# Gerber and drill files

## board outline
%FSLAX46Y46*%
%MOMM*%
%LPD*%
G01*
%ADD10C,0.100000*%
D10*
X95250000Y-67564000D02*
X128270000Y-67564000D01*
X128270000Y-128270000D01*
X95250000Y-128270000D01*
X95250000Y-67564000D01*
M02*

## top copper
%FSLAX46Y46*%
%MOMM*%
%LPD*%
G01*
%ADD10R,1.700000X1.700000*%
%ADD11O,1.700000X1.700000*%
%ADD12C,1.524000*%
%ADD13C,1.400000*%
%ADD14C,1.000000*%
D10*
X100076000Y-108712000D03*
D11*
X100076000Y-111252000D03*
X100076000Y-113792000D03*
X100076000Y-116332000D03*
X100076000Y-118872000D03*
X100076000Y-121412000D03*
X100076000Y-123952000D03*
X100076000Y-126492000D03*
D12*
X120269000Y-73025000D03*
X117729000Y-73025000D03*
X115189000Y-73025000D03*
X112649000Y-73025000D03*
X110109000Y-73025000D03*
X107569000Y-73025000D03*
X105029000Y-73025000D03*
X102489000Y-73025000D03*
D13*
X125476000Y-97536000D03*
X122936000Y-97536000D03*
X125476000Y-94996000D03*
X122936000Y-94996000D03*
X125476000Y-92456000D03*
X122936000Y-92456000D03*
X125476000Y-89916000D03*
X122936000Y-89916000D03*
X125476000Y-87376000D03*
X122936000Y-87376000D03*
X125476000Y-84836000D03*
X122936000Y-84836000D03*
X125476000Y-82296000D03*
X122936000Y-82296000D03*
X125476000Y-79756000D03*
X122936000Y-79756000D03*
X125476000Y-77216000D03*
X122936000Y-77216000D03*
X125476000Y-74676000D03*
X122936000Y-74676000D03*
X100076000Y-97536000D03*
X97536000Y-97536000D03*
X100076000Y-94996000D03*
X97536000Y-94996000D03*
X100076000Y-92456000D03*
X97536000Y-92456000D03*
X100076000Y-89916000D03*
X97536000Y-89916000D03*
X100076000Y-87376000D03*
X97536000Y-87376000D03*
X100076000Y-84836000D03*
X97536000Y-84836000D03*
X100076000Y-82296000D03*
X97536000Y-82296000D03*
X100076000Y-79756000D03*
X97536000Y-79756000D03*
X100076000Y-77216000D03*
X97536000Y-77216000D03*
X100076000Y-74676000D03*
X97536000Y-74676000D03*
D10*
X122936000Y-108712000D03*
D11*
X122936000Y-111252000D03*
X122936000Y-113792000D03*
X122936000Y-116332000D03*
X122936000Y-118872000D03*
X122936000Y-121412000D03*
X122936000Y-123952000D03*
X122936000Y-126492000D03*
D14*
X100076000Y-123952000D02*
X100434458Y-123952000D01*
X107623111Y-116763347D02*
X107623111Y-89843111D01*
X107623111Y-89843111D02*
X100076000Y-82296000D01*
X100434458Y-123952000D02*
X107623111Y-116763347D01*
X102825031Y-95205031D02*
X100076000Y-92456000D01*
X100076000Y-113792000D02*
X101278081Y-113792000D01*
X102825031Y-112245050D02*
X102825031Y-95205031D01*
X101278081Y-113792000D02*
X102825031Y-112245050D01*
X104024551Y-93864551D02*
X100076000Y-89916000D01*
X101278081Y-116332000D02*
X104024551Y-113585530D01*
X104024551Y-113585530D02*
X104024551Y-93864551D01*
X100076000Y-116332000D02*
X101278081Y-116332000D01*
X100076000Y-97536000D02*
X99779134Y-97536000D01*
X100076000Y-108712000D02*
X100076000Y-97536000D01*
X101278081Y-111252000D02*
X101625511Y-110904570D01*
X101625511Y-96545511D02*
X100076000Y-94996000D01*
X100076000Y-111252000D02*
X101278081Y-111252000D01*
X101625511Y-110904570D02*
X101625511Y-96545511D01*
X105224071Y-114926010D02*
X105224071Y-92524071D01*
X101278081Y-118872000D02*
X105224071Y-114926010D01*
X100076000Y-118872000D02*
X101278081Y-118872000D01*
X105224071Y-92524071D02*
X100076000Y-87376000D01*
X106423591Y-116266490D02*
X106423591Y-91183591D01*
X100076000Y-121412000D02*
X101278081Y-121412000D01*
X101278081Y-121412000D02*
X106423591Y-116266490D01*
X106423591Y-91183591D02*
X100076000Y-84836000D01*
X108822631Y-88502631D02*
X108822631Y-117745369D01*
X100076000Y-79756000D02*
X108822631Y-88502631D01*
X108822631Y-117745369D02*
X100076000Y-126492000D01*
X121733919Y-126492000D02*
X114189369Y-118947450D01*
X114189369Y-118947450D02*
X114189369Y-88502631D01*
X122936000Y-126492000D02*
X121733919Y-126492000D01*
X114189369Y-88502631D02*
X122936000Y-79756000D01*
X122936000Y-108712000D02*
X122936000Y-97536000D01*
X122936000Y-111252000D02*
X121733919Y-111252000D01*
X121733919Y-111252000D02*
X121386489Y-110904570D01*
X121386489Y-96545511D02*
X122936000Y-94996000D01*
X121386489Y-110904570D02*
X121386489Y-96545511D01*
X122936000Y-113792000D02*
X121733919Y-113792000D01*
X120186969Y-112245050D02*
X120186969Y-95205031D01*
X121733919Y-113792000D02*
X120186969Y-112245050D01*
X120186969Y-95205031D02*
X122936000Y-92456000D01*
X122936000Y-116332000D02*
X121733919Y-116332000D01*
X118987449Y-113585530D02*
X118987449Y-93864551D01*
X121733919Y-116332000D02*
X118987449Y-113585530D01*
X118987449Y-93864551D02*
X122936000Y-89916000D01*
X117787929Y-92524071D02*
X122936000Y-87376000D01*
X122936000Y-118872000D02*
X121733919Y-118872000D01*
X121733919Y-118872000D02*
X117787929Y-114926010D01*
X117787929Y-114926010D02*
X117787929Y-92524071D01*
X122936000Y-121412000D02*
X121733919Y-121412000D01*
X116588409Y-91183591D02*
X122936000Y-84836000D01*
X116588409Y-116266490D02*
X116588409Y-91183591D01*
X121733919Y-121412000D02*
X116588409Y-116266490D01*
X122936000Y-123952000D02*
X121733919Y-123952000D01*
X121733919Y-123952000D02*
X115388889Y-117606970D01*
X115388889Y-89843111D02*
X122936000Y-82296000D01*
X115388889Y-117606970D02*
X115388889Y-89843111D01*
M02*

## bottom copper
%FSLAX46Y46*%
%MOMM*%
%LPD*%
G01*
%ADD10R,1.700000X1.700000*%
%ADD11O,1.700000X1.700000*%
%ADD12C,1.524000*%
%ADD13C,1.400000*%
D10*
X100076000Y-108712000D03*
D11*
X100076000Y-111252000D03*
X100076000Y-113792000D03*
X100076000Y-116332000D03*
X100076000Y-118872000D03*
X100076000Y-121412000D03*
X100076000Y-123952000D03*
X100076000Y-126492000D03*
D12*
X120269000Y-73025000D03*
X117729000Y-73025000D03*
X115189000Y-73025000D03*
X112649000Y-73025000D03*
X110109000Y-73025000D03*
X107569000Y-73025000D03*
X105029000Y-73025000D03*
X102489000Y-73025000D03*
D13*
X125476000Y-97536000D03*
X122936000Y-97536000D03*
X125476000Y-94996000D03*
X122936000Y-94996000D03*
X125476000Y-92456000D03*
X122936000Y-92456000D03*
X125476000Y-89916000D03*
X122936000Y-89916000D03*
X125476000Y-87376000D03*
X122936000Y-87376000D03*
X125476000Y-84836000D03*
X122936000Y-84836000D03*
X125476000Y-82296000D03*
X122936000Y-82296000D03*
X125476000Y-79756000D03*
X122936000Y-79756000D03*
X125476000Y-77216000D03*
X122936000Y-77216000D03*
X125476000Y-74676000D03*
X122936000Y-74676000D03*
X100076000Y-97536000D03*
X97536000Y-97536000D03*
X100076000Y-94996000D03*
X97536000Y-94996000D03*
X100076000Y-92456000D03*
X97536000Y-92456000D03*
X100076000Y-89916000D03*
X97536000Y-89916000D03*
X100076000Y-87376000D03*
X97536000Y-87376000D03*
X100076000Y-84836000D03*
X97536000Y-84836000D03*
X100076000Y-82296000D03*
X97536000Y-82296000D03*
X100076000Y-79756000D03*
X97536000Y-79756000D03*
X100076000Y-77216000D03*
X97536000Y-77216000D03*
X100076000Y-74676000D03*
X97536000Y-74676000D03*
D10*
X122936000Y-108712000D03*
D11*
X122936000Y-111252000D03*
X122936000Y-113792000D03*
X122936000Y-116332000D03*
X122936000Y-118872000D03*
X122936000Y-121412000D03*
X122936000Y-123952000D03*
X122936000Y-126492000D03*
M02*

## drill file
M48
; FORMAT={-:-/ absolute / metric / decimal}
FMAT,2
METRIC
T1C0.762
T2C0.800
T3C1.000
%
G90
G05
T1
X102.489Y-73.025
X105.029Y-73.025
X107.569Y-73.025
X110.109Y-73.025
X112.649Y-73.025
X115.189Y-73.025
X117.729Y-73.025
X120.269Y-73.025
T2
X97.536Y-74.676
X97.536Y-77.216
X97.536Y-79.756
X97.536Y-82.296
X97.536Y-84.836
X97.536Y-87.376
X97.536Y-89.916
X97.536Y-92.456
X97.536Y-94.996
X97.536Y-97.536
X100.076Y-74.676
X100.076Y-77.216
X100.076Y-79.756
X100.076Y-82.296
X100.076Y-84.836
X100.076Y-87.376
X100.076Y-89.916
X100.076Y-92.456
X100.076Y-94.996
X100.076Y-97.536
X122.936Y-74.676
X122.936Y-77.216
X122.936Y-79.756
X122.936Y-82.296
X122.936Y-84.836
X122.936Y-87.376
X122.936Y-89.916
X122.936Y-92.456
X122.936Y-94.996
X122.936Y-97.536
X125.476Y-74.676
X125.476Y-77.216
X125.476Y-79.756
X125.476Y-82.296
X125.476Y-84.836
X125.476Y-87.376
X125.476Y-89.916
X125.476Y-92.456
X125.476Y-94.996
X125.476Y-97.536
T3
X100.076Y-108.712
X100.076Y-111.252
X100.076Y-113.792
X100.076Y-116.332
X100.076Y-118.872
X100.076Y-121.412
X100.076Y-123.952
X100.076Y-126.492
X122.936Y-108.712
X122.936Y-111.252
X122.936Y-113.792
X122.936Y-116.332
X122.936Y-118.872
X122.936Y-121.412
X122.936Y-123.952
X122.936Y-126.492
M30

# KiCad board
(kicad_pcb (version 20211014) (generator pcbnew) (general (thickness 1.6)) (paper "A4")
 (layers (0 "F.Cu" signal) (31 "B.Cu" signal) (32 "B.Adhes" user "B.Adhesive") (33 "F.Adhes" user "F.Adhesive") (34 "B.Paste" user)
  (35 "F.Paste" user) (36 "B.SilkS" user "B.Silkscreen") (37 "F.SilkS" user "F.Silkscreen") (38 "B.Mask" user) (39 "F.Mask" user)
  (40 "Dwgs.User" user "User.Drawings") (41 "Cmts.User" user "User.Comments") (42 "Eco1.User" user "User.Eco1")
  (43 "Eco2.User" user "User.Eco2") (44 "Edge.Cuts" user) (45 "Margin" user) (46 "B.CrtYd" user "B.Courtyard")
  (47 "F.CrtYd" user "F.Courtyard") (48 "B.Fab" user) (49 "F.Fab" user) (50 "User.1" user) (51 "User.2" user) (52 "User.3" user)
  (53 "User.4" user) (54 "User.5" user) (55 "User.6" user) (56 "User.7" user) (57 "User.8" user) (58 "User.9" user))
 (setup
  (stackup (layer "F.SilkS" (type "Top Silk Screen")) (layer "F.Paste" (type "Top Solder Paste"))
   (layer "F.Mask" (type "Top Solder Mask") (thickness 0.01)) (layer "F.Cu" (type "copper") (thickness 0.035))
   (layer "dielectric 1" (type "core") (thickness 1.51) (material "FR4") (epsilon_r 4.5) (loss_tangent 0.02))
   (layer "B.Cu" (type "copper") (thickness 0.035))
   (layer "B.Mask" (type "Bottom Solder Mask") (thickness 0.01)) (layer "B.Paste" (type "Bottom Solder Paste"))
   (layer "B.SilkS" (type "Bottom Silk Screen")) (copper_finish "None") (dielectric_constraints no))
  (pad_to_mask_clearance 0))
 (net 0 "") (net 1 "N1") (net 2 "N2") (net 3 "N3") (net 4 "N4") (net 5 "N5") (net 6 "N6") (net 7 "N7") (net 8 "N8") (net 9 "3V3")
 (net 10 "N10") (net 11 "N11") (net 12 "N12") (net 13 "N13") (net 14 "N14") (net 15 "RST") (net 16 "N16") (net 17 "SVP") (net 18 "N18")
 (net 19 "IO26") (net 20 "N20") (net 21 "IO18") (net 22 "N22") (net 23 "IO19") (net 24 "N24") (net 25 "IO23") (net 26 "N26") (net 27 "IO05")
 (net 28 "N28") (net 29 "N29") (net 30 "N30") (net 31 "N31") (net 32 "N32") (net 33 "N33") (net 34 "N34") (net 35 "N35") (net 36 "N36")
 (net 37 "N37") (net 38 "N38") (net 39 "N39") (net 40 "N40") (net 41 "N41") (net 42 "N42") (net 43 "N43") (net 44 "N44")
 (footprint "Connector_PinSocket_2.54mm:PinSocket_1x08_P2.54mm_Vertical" (layer "F.Cu") (at 100.076 108.712)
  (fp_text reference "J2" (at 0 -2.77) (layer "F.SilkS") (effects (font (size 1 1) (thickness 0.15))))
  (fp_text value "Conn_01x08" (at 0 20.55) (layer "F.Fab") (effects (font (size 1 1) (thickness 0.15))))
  (pad "1" thru_hole rect (at 0 0) (size 1.7 1.7) (drill 1) (layers *.Cu *.Mask) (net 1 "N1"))
  (pad "2" thru_hole oval (at 0 2.54) (size 1.7 1.7) (drill 1) (layers *.Cu *.Mask) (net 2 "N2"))
  (pad "3" thru_hole oval (at 0 5.08) (size 1.7 1.7) (drill 1) (layers *.Cu *.Mask) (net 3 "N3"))
  (pad "4" thru_hole oval (at 0 7.62) (size 1.7 1.7) (drill 1) (layers *.Cu *.Mask) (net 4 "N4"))
  (pad "5" thru_hole oval (at 0 10.16) (size 1.7 1.7) (drill 1) (layers *.Cu *.Mask) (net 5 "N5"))
  (pad "6" thru_hole oval (at 0 12.7) (size 1.7 1.7) (drill 1) (layers *.Cu *.Mask) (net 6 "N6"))
  (pad "7" thru_hole oval (at 0 15.24) (size 1.7 1.7) (drill 1) (layers *.Cu *.Mask) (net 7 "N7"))
  (pad "8" thru_hole oval (at 0 17.78) (size 1.7 1.7) (drill 1) (layers *.Cu *.Mask) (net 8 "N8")))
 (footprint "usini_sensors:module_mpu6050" (layer "F.Cu") (at 102.489 73.025 -90)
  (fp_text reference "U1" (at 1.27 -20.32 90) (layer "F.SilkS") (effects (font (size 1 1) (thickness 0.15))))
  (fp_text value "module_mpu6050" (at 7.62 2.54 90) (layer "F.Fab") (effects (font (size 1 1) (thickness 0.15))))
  (pad "1" thru_hole circle locked (at 0 -17.78 270) (size 1.524 1.524) (drill 0.762) (layers *.Cu *.Mask) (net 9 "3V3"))
  (pad "2" thru_hole circle locked (at 0 -15.24 270) (size 1.524 1.524) (drill 0.762) (layers *.Cu *.Mask) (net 7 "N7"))
  (pad "3" thru_hole circle locked (at 0 -12.7 270) (size 1.524 1.524) (drill 0.762) (layers *.Cu *.Mask) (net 3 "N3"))
  (pad "4" thru_hole circle locked (at 0 -10.16 270) (size 1.524 1.524) (drill 0.762) (layers *.Cu *.Mask) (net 4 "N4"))
  (pad "5" thru_hole circle locked (at 0 -7.62 270) (size 1.524 1.524) (drill 0.762) (layers *.Cu *.Mask) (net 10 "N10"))
  (pad "6" thru_hole circle locked (at 0 -5.08 270) (size 1.524 1.524) (drill 0.762) (layers *.Cu *.Mask) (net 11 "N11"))
  (pad "7" thru_hole circle locked (at 0 -2.54 270) (size 1.524 1.524) (drill 0.762) (layers *.Cu *.Mask) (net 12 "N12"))
  (pad "8" thru_hole circle locked (at 0 0 270) (size 1.524 1.524) (drill 0.762) (layers *.Cu *.Mask) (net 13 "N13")))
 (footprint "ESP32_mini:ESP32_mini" (layer "F.Cu") (at 111.506 86.106 180)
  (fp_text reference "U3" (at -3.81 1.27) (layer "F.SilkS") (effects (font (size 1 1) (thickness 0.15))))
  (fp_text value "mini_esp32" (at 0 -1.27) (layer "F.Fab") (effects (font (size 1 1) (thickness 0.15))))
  (pad "1" thru_hole circle locked (at -13.97 -11.43 90) (size 1.4 1.4) (drill 0.8) (layers *.Cu *.Mask) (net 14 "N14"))
  (pad "2" thru_hole circle locked (at -11.43 -11.43 90) (size 1.4 1.4) (drill 0.8) (layers *.Cu *.Mask) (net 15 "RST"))
  (pad "3" thru_hole circle locked (at -13.97 -8.89 90) (size 1.4 1.4) (drill 0.8) (layers *.Cu *.Mask) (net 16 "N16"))
  (pad "4" thru_hole circle locked (at -11.43 -8.89 90) (size 1.4 1.4) (drill 0.8) (layers *.Cu *.Mask) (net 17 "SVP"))
  (pad "5" thru_hole circle locked (at -13.97 -6.35 90) (size 1.4 1.4) (drill 0.8) (layers *.Cu *.Mask) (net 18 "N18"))
  (pad "6" thru_hole circle locked (at -11.43 -6.35 90) (size 1.4 1.4) (drill 0.8) (layers *.Cu *.Mask) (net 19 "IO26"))
  (pad "7" thru_hole circle locked (at -13.97 -3.81 90) (size 1.4 1.4) (drill 0.8) (layers *.Cu *.Mask) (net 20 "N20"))
  (pad "8" thru_hole circle locked (at -11.43 -3.81 90) (size 1.4 1.4) (drill 0.8) (layers *.Cu *.Mask) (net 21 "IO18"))
  (pad "9" thru_hole circle locked (at -13.97 -1.27 90) (size 1.4 1.4) (drill 0.8) (layers *.Cu *.Mask) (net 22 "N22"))
  (pad "10" thru_hole circle locked (at -11.43 -1.27 90) (size 1.4 1.4) (drill 0.8) (layers *.Cu *.Mask) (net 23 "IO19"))
  (pad "11" thru_hole circle locked (at -13.97 1.27 90) (size 1.4 1.4) (drill 0.8) (layers *.Cu *.Mask) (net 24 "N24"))
  (pad "12" thru_hole circle locked (at -11.43 1.27 90) (size 1.4 1.4) (drill 0.8) (layers *.Cu *.Mask) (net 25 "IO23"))
  (pad "13" thru_hole circle locked (at -13.97 3.81 90) (size 1.4 1.4) (drill 0.8) (layers *.Cu *.Mask) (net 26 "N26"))
  (pad "14" thru_hole circle locked (at -11.43 3.81 90) (size 1.4 1.4) (drill 0.8) (layers *.Cu *.Mask) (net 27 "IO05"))
  (pad "15" thru_hole circle locked (at -13.97 6.35 90) (size 1.4 1.4) (drill 0.8) (layers *.Cu *.Mask) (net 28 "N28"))
  (pad "16" thru_hole circle locked (at -11.43 6.35 90) (size 1.4 1.4) (drill 0.8) (layers *.Cu *.Mask) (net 9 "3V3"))
  (pad "17" thru_hole circle locked (at -13.97 8.89 90) (size 1.4 1.4) (drill 0.8) (layers *.Cu *.Mask) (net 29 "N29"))
  (pad "18" thru_hole circle locked (at -11.43 8.89 90) (size 1.4 1.4) (drill 0.8) (layers *.Cu *.Mask) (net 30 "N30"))
  (pad "19" thru_hole circle locked (at -13.97 11.43 90) (size 1.4 1.4) (drill 0.8) (layers *.Cu *.Mask) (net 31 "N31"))
  (pad "20" thru_hole circle locked (at -11.43 11.43 90) (size 1.4 1.4) (drill 0.8) (layers *.Cu *.Mask) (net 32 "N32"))
  (pad "21" thru_hole circle locked (at 11.43 -11.43 90) (size 1.4 1.4) (drill 0.8) (layers *.Cu *.Mask) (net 1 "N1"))
  (pad "22" thru_hole circle locked (at 13.97 -11.43 90) (size 1.4 1.4) (drill 0.8) (layers *.Cu *.Mask) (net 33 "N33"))
  (pad "23" thru_hole circle locked (at 11.43 -8.89 90) (size 1.4 1.4) (drill 0.8) (layers *.Cu *.Mask) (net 2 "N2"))
  (pad "24" thru_hole circle locked (at 13.97 -8.89 90) (size 1.4 1.4) (drill 0.8) (layers *.Cu *.Mask) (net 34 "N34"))
  (pad "25" thru_hole circle locked (at 11.43 -6.35 90) (size 1.4 1.4) (drill 0.8) (layers *.Cu *.Mask) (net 3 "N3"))
  (pad "26" thru_hole circle locked (at 13.97 -6.35 90) (size 1.4 1.4) (drill 0.8) (layers *.Cu *.Mask) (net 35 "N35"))
  (pad "27" thru_hole circle locked (at 11.43 -3.81 90) (size 1.4 1.4) (drill 0.8) (layers *.Cu *.Mask) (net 4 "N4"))
  (pad "28" thru_hole circle locked (at 13.97 -3.81 90) (size 1.4 1.4) (drill 0.8) (layers *.Cu *.Mask) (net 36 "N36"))
  (pad "29" thru_hole circle locked (at 11.43 -1.27 90) (size 1.4 1.4) (drill 0.8) (layers *.Cu *.Mask) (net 5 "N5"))
  (pad "30" thru_hole circle locked (at 13.97 -1.27 90) (size 1.4 1.4) (drill 0.8) (layers *.Cu *.Mask) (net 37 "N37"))
  (pad "31" thru_hole circle locked (at 11.43 1.27 90) (size 1.4 1.4) (drill 0.8) (layers *.Cu *.Mask) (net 6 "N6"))
  (pad "32" thru_hole circle locked (at 13.97 1.27 90) (size 1.4 1.4) (drill 0.8) (layers *.Cu *.Mask) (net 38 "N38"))
  (pad "33" thru_hole circle locked (at 11.43 3.81 90) (size 1.4 1.4) (drill 0.8) (layers *.Cu *.Mask) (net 7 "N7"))
  (pad "34" thru_hole circle locked (at 13.97 3.81 90) (size 1.4 1.4) (drill 0.8) (layers *.Cu *.Mask) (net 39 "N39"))
  (pad "35" thru_hole circle locked (at 11.43 6.35 90) (size 1.4 1.4) (drill 0.8) (layers *.Cu *.Mask) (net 8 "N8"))
  (pad "36" thru_hole circle locked (at 13.97 6.35 90) (size 1.4 1.4) (drill 0.8) (layers *.Cu *.Mask) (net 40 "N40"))
  (pad "37" thru_hole circle locked (at 11.43 8.89 90) (size 1.4 1.4) (drill 0.8) (layers *.Cu *.Mask) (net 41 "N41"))
  (pad "38" thru_hole circle locked (at 13.97 8.89 90) (size 1.4 1.4) (drill 0.8) (layers *.Cu *.Mask) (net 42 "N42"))
  (pad "39" thru_hole circle locked (at 11.43 11.43 90) (size 1.4 1.4) (drill 0.8) (layers *.Cu *.Mask) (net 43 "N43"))
  (pad "40" thru_hole circle locked (at 13.97 11.43 90) (size 1.4 1.4) (drill 0.8) (layers *.Cu *.Mask) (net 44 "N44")))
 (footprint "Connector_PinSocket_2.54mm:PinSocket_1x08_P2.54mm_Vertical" (layer "F.Cu") (at 122.936 108.712)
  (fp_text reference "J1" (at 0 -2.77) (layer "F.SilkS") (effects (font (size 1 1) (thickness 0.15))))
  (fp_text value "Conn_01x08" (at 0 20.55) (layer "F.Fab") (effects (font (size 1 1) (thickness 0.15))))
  (pad "1" thru_hole rect (at 0 0) (size 1.7 1.7) (drill 1) (layers *.Cu *.Mask) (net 15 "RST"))
  (pad "2" thru_hole oval (at 0 2.54) (size 1.7 1.7) (drill 1) (layers *.Cu *.Mask) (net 17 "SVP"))
  (pad "3" thru_hole oval (at 0 5.08) (size 1.7 1.7) (drill 1) (layers *.Cu *.Mask) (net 19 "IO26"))
  (pad "4" thru_hole oval (at 0 7.62) (size 1.7 1.7) (drill 1) (layers *.Cu *.Mask) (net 21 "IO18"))
  (pad "5" thru_hole oval (at 0 10.16) (size 1.7 1.7) (drill 1) (layers *.Cu *.Mask) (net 23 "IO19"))
  (pad "6" thru_hole oval (at 0 12.7) (size 1.7 1.7) (drill 1) (layers *.Cu *.Mask) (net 25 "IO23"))
  (pad "7" thru_hole oval (at 0 15.24) (size 1.7 1.7) (drill 1) (layers *.Cu *.Mask) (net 27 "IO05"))
  (pad "8" thru_hole oval (at 0 17.78) (size 1.7 1.7) (drill 1) (layers *.Cu *.Mask) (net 9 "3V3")))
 (gr_rect (start 95.25 67.564) (end 128.27 128.27) (layer "Edge.Cuts") (width 0.1) (fill none))
 (segment (start 100.076 123.952) (end 100.434458 123.952) (width 1) (layer "F.Cu") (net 7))
 (segment (start 107.623111 116.763347) (end 107.623111 89.843111) (width 1) (layer "F.Cu") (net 7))
 (segment (start 107.623111 89.843111) (end 100.076 82.296) (width 1) (layer "F.Cu") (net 7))
 (segment (start 100.434458 123.952) (end 107.623111 116.763347) (width 1) (layer "F.Cu") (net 7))
 (segment (start 102.825031 95.205031) (end 100.076 92.456) (width 1) (layer "F.Cu") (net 3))
 (segment (start 100.076 113.792) (end 101.278081 113.792) (width 1) (layer "F.Cu") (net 3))
 (segment (start 102.825031 112.24505) (end 102.825031 95.205031) (width 1) (layer "F.Cu") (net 3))
 (segment (start 101.278081 113.792) (end 102.825031 112.24505) (width 1) (layer "F.Cu") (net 3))
 (segment (start 104.024551 93.864551) (end 100.076 89.916) (width 1) (layer "F.Cu") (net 4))
 (segment (start 101.278081 116.332) (end 104.024551 113.58553) (width 1) (layer "F.Cu") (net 4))
 (segment (start 104.024551 113.58553) (end 104.024551 93.864551) (width 1) (layer "F.Cu") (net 4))
 (segment (start 100.076 116.332) (end 101.278081 116.332) (width 1) (layer "F.Cu") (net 4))
 (segment (start 100.076 97.536) (end 99.779134 97.536) (width 1) (layer "F.Cu") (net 1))
 (segment (start 100.076 108.712) (end 100.076 97.536) (width 1) (layer "F.Cu") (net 1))
 (segment (start 101.278081 111.252) (end 101.625511 110.90457) (width 1) (layer "F.Cu") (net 2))
 (segment (start 101.625511 96.545511) (end 100.076 94.996) (width 1) (layer "F.Cu") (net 2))
 (segment (start 100.076 111.252) (end 101.278081 111.252) (width 1) (layer "F.Cu") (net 2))
 (segment (start 101.625511 110.90457) (end 101.625511 96.545511) (width 1) (layer "F.Cu") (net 2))
 (segment (start 105.224071 114.92601) (end 105.224071 92.524071) (width 1) (layer "F.Cu") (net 5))
 (segment (start 101.278081 118.872) (end 105.224071 114.92601) (width 1) (layer "F.Cu") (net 5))
 (segment (start 100.076 118.872) (end 101.278081 118.872) (width 1) (layer "F.Cu") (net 5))
 (segment (start 105.224071 92.524071) (end 100.076 87.376) (width 1) (layer "F.Cu") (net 5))
 (segment (start 106.423591 116.26649) (end 106.423591 91.183591) (width 1) (layer "F.Cu") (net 6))
 (segment (start 100.076 121.412) (end 101.278081 121.412) (width 1) (layer "F.Cu") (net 6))
 (segment (start 101.278081 121.412) (end 106.423591 116.26649) (width 1) (layer "F.Cu") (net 6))
 (segment (start 106.423591 91.183591) (end 100.076 84.836) (width 1) (layer "F.Cu") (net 6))
 (segment (start 108.822631 88.502631) (end 108.822631 117.745369) (width 1) (layer "F.Cu") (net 8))
 (segment (start 100.076 79.756) (end 108.822631 88.502631) (width 1) (layer "F.Cu") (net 8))
 (segment (start 108.822631 117.745369) (end 100.076 126.492) (width 1) (layer "F.Cu") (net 8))
 (segment (start 121.733919 126.492) (end 114.189369 118.94745) (width 1) (layer "F.Cu") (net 9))
 (segment (start 114.189369 118.94745) (end 114.189369 88.502631) (width 1) (layer "F.Cu") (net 9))
 (segment (start 122.936 126.492) (end 121.733919 126.492) (width 1) (layer "F.Cu") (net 9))
 (segment (start 114.189369 88.502631) (end 122.936 79.756) (width 1) (layer "F.Cu") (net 9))
 (segment (start 122.936 108.712) (end 122.936 97.536) (width 1) (layer "F.Cu") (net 15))
 (segment (start 122.936 111.252) (end 121.733919 111.252) (width 1) (layer "F.Cu") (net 17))
 (segment (start 121.733919 111.252) (end 121.386489 110.90457) (width 1) (layer "F.Cu") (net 17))
 (segment (start 121.386489 96.545511) (end 122.936 94.996) (width 1) (layer "F.Cu") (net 17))
 (segment (start 121.386489 110.90457) (end 121.386489 96.545511) (width 1) (layer "F.Cu") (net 17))
 (segment (start 122.936 113.792) (end 121.733919 113.792) (width 1) (layer "F.Cu") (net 19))
 (segment (start 120.186969 112.24505) (end 120.186969 95.205031) (width 1) (layer "F.Cu") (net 19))
 (segment (start 121.733919 113.792) (end 120.186969 112.24505) (width 1) (layer "F.Cu") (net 19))
 (segment (start 120.186969 95.205031) (end 122.936 92.456) (width 1) (layer "F.Cu") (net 19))
 (segment (start 122.936 116.332) (end 121.733919 116.332) (width 1) (layer "F.Cu") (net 21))
 (segment (start 118.987449 113.58553) (end 118.987449 93.864551) (width 1) (layer "F.Cu") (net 21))
 (segment (start 121.733919 116.332) (end 118.987449 113.58553) (width 1) (layer "F.Cu") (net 21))
 (segment (start 118.987449 93.864551) (end 122.936 89.916) (width 1) (layer "F.Cu") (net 21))
 (segment (start 117.787929 92.524071) (end 122.936 87.376) (width 1) (layer "F.Cu") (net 23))
 (segment (start 122.936 118.872) (end 121.733919 118.872) (width 1) (layer "F.Cu") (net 23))
 (segment (start 121.733919 118.872) (end 117.787929 114.92601) (width 1) (layer "F.Cu") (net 23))
 (segment (start 117.787929 114.92601) (end 117.787929 92.524071) (width 1) (layer "F.Cu") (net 23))
 (segment (start 122.936 121.412) (end 121.733919 121.412) (width 1) (layer "F.Cu") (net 25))
 (segment (start 116.588409 91.183591) (end 122.936 84.836) (width 1) (layer "F.Cu") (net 25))
 (segment (start 116.588409 116.26649) (end 116.588409 91.183591) (width 1) (layer "F.Cu") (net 25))
 (segment (start 121.733919 121.412) (end 116.588409 116.26649) (width 1) (layer "F.Cu") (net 25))
 (segment (start 122.936 123.952) (end 121.733919 123.952) (width 1) (layer "F.Cu") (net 27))
 (segment (start 121.733919 123.952) (end 115.388889 117.60697) (width 1) (layer "F.Cu") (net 27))
 (segment (start 115.388889 89.843111) (end 122.936 82.296) (width 1) (layer "F.Cu") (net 27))
 (segment (start 115.388889 117.60697) (end 115.388889 89.843111) (width 1) (layer "F.Cu") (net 27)))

